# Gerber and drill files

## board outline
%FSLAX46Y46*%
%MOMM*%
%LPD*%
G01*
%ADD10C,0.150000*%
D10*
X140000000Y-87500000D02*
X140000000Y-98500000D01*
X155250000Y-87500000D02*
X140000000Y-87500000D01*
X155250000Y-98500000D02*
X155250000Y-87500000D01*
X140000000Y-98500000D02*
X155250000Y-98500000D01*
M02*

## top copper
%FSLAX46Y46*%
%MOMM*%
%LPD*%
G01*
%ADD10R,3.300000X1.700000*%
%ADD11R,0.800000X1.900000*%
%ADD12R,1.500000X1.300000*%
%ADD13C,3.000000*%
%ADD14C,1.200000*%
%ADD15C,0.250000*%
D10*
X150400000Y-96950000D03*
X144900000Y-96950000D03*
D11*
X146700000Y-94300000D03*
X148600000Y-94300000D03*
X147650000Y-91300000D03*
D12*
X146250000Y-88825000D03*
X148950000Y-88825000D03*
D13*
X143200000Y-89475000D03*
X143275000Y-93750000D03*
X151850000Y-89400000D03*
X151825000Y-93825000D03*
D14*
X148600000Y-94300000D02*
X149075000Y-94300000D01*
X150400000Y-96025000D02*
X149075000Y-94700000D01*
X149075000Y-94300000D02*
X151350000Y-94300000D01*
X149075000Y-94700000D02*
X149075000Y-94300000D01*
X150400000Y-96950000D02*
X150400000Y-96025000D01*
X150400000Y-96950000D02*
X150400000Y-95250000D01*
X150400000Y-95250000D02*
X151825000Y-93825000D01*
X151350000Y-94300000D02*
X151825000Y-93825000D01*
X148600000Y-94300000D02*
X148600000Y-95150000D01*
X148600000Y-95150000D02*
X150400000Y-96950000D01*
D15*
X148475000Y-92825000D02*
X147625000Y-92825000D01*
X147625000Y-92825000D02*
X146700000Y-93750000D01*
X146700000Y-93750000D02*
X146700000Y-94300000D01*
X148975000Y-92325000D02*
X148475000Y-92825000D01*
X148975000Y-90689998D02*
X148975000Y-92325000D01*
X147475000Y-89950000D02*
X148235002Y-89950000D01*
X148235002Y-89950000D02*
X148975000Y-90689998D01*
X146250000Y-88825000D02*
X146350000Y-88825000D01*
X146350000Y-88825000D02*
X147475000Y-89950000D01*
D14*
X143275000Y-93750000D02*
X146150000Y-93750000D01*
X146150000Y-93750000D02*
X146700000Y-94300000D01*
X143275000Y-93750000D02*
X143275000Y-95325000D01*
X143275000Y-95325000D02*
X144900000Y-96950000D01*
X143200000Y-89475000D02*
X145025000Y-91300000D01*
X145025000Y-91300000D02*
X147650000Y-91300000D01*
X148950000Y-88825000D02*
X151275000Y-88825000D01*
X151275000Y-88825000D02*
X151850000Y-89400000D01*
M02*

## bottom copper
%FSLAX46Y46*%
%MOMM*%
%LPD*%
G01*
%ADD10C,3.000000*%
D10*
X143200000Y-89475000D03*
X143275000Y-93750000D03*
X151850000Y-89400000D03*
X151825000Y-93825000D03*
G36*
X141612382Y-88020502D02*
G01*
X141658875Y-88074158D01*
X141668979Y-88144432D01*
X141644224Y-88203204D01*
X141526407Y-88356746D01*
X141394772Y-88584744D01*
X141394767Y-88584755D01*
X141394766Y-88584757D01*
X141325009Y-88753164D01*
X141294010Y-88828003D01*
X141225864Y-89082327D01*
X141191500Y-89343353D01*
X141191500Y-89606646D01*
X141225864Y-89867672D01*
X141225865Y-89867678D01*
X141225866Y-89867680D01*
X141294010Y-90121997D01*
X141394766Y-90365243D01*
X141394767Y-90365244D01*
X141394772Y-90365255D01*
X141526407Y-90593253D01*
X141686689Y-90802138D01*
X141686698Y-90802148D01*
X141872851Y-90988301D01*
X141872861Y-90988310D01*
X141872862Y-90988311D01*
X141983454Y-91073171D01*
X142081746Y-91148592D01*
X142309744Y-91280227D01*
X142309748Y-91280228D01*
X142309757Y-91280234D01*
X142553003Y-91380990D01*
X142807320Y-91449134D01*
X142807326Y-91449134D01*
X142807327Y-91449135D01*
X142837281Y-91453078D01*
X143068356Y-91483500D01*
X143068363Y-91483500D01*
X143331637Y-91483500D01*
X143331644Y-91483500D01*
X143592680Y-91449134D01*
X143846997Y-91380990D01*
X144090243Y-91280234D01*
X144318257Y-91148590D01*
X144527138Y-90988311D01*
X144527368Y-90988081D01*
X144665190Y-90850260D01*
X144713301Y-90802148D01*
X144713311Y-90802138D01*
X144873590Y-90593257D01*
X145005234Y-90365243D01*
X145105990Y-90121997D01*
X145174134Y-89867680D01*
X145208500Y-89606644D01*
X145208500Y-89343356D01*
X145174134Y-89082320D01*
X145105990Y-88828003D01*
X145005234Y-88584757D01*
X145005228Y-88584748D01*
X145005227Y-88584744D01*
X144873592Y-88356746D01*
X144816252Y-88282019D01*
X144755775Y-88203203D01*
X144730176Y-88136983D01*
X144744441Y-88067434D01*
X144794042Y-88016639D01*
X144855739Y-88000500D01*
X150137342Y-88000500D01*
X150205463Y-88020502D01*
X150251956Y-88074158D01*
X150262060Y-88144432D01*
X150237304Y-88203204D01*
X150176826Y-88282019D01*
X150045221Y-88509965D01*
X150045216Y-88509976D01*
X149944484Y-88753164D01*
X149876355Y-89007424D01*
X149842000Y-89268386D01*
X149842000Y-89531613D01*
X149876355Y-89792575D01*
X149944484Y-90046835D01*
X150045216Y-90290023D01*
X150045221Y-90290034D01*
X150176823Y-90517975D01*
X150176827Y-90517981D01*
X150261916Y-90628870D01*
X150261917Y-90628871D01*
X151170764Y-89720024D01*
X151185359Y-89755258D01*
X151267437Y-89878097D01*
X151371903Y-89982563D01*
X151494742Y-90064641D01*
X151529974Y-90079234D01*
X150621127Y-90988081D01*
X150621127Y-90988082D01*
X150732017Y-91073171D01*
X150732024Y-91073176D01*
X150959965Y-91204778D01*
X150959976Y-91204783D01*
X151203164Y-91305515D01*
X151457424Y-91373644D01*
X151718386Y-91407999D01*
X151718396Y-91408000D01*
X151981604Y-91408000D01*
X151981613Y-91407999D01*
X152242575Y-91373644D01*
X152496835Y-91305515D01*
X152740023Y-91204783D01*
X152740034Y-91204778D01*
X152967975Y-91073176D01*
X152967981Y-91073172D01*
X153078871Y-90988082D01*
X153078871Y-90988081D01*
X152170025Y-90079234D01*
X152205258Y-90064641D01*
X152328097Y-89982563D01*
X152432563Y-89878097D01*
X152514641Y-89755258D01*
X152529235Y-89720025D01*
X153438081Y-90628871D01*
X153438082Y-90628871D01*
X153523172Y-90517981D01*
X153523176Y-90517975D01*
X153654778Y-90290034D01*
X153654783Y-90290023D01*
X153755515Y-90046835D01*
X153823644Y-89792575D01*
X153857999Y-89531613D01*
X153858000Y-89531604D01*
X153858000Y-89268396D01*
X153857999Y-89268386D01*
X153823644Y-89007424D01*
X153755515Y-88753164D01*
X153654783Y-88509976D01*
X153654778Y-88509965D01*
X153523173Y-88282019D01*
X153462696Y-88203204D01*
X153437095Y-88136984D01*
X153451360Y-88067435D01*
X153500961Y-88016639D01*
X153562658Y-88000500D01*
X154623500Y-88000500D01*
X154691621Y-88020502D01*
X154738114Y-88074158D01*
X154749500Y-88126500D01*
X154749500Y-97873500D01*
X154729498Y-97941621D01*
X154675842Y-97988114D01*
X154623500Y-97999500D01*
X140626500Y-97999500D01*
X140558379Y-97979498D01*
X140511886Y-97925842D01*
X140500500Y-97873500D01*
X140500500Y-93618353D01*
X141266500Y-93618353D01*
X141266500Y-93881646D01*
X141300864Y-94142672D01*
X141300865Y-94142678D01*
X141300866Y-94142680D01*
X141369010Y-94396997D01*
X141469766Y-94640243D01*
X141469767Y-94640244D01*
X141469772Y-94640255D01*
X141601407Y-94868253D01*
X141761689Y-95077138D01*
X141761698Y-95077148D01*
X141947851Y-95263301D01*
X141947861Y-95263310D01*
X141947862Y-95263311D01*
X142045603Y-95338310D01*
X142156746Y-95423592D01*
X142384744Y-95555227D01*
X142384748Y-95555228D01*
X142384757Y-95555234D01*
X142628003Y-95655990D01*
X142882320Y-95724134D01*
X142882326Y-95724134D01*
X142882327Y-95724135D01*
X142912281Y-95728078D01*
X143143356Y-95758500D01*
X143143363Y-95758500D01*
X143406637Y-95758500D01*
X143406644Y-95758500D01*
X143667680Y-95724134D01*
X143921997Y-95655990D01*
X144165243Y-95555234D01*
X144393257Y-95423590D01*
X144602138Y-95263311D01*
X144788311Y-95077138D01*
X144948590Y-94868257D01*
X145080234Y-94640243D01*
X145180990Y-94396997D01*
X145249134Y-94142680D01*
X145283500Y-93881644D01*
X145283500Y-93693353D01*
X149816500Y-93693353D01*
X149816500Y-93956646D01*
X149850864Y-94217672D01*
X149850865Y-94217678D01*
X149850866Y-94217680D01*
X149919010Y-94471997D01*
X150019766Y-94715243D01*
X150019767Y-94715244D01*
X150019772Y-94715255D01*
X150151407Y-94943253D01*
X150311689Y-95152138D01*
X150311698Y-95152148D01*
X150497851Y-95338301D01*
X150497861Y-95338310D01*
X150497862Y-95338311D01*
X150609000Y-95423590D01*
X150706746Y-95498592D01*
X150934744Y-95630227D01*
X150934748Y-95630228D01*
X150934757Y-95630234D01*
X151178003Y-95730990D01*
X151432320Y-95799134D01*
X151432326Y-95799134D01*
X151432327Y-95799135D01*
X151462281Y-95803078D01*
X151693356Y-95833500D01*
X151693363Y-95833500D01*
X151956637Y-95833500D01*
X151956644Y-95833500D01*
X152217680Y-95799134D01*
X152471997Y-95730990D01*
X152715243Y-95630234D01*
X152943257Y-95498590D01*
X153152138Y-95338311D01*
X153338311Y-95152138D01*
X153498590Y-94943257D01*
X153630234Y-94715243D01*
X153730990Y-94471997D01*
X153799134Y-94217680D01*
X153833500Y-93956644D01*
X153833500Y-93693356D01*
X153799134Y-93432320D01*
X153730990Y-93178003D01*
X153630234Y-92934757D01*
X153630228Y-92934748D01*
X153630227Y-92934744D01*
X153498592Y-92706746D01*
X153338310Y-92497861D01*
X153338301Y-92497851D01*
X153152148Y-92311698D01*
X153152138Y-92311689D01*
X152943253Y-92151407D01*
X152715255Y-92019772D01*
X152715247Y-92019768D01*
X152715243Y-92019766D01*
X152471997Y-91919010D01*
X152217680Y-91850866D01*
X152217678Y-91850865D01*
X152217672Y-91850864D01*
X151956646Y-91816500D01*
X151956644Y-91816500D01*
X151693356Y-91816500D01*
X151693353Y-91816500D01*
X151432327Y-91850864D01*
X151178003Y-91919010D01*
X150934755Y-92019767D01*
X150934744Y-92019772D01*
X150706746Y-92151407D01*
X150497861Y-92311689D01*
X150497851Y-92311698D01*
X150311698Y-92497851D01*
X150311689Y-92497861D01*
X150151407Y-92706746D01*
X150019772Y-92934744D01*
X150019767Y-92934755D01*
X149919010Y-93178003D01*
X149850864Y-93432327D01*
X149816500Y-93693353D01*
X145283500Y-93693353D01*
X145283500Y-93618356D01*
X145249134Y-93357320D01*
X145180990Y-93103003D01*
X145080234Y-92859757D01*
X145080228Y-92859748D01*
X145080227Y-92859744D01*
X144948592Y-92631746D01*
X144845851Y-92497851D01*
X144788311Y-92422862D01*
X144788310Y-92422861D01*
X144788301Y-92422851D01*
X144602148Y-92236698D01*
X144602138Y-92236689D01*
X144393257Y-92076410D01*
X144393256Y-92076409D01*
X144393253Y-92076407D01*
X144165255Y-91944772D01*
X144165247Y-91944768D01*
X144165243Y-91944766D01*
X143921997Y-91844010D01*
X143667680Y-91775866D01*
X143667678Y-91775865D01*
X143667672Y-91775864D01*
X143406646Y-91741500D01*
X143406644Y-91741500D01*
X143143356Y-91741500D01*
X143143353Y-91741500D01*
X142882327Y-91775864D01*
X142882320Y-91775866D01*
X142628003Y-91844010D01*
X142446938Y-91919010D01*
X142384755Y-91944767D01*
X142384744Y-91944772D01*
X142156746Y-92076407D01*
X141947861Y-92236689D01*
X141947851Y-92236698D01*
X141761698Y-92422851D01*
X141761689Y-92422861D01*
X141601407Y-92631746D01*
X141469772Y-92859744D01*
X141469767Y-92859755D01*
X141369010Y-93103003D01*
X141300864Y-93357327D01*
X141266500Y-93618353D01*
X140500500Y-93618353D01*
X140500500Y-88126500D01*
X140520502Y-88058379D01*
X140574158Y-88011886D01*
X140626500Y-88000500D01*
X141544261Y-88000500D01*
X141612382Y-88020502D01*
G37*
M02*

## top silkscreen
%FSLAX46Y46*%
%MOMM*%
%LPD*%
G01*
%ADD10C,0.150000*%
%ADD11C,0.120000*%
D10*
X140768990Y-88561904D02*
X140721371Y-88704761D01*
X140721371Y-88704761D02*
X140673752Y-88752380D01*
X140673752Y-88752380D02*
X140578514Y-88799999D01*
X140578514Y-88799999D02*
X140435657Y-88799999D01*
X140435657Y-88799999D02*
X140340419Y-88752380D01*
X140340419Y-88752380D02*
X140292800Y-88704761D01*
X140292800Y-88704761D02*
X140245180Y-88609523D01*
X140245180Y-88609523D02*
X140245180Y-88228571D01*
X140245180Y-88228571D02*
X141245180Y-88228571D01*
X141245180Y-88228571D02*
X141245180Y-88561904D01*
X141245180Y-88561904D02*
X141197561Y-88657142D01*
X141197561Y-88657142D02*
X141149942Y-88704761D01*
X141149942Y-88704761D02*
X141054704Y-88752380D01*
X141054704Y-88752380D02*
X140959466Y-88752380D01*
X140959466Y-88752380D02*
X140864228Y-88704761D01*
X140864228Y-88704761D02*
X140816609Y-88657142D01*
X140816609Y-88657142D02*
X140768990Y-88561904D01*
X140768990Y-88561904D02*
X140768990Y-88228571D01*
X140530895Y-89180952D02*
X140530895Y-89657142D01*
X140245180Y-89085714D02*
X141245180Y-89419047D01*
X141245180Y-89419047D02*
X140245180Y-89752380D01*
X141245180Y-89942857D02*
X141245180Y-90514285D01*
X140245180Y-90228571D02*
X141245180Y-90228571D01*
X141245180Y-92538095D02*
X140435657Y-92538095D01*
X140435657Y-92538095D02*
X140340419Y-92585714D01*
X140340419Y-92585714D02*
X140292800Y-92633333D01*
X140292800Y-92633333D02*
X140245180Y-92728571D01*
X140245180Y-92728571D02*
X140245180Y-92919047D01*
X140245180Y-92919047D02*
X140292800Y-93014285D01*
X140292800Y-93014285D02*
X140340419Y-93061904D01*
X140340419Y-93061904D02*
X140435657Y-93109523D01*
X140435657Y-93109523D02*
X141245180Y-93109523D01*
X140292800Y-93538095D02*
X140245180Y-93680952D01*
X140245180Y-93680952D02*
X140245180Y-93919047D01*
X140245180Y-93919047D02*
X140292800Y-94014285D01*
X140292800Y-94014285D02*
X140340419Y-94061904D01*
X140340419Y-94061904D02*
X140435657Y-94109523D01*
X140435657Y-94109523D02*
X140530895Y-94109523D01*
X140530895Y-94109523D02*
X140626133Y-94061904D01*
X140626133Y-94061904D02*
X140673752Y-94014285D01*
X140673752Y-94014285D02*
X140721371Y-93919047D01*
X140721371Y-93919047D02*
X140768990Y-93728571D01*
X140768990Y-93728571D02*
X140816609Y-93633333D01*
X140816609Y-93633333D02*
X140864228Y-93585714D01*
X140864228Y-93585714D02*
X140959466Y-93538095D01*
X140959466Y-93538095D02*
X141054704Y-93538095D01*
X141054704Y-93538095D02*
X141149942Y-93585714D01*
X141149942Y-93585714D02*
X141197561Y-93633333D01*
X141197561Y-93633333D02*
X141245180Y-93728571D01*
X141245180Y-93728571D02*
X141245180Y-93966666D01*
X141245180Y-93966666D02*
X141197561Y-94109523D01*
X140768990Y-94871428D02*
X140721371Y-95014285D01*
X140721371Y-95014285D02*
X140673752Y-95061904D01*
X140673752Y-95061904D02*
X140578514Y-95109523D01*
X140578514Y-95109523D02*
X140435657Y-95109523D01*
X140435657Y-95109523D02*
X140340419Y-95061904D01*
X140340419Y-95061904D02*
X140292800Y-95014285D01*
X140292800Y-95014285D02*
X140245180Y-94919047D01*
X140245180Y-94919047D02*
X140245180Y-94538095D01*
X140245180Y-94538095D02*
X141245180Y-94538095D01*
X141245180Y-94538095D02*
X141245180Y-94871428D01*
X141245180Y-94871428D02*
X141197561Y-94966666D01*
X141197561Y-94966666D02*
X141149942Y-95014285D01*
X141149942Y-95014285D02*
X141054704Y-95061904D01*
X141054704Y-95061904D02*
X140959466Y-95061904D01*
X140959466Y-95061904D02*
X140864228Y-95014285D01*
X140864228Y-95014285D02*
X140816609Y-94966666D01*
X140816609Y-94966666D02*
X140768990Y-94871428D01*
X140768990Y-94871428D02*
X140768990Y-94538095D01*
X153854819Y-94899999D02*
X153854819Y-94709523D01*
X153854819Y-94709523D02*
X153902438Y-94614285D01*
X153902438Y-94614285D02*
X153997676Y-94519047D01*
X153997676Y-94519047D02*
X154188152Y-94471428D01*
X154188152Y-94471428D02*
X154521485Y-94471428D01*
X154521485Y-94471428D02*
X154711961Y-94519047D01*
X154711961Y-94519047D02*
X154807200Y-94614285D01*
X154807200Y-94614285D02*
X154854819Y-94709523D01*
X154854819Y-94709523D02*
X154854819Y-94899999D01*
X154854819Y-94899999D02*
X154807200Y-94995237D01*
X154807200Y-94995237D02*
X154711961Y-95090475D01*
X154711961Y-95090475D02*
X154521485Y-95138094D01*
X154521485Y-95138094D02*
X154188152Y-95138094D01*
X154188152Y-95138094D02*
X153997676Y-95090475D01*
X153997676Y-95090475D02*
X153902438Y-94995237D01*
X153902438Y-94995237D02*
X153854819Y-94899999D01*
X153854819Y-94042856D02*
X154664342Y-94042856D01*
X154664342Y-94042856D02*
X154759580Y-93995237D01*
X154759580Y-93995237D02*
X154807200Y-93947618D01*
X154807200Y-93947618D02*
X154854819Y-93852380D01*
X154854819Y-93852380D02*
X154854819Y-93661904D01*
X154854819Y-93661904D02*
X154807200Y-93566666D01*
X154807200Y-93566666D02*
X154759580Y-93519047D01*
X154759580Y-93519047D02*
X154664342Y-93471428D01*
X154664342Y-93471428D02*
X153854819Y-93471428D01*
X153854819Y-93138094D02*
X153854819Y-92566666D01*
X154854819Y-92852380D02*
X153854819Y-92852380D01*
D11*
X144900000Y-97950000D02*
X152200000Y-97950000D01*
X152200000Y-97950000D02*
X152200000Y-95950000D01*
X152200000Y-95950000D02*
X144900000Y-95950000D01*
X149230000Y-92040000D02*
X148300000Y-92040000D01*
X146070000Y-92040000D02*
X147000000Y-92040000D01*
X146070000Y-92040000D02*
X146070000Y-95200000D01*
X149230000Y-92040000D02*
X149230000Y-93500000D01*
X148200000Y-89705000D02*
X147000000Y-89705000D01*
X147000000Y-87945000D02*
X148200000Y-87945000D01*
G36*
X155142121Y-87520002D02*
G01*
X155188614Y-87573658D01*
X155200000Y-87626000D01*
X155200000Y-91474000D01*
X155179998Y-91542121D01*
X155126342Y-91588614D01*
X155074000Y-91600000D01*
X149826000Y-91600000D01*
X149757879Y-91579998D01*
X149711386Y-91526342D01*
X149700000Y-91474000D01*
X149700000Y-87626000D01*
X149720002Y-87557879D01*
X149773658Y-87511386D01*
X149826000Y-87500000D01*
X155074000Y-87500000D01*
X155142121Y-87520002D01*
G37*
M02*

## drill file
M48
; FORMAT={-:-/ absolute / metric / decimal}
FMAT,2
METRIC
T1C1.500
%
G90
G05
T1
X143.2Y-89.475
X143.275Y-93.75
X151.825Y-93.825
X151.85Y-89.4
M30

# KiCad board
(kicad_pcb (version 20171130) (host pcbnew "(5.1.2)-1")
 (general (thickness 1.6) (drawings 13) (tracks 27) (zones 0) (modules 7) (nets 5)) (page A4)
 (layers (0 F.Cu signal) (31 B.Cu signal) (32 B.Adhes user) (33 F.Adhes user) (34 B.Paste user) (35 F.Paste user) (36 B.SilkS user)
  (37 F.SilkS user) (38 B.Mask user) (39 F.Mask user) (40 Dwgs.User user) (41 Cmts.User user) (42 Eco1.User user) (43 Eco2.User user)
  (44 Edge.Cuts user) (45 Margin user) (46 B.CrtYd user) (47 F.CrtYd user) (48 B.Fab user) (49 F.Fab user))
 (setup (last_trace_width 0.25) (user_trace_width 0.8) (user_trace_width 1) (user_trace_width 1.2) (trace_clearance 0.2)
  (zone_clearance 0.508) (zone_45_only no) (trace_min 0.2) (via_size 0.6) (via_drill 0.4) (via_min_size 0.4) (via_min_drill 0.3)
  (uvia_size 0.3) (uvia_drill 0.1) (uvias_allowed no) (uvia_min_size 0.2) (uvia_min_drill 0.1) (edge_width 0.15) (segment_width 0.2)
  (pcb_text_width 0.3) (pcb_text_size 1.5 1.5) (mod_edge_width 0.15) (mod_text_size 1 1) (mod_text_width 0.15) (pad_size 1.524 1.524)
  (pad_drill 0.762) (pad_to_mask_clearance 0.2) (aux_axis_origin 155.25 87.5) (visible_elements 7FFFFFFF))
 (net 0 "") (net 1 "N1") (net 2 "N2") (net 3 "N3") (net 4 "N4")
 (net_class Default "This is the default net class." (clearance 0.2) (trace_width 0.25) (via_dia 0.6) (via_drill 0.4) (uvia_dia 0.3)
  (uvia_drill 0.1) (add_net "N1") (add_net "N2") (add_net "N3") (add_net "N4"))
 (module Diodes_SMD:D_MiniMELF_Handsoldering (layer F.Cu) (at 147.65 96.95 180)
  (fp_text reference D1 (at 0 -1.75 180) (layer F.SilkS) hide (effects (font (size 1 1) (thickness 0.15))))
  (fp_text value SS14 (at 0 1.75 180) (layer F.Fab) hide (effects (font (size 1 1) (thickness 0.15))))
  (fp_line (start 2.75 -1) (end -4.55 -1) (layer F.SilkS) (width 0.12))
  (fp_line (start -4.55 -1) (end -4.55 1) (layer F.SilkS) (width 0.12))
  (fp_line (start -4.55 1) (end 2.75 1) (layer F.SilkS) (width 0.12))
  (pad 1 smd rect (at -2.75 0 180) (size 3.3 1.7) (layers F.Cu F.Paste F.Mask) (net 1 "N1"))
  (pad 2 smd rect (at 2.75 0 180) (size 3.3 1.7) (layers F.Cu F.Paste F.Mask) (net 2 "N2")))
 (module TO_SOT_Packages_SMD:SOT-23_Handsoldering (layer F.Cu) (at 147.65 92.8 90)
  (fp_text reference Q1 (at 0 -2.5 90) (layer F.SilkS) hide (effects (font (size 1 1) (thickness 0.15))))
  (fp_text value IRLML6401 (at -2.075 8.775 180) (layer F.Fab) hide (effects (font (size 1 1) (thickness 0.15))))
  (fp_line (start 0.76 1.58) (end 0.76 0.65) (layer F.SilkS) (width 0.12))
  (fp_line (start 0.76 -1.58) (end 0.76 -0.65) (layer F.SilkS) (width 0.12))
  (fp_line (start 0.76 -1.58) (end -2.4 -1.58) (layer F.SilkS) (width 0.12))
  (fp_line (start 0.76 1.58) (end -0.7 1.58) (layer F.SilkS) (width 0.12))
  (pad 1 smd rect (at -1.5 -0.95 90) (size 1.9 0.8) (layers F.Cu F.Paste F.Mask) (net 2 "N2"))
  (pad 2 smd rect (at -1.5 0.95 90) (size 1.9 0.8) (layers F.Cu F.Paste F.Mask) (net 1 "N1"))
  (pad 3 smd rect (at 1.5 0 90) (size 1.9 0.8) (layers F.Cu F.Paste F.Mask) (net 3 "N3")))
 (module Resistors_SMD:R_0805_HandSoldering (layer F.Cu) (at 147.6 88.825)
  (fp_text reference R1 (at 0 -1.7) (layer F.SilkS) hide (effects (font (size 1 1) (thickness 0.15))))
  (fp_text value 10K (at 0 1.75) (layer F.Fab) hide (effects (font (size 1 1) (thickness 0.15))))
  (fp_line (start 0.6 0.88) (end -0.6 0.88) (layer F.SilkS) (width 0.12))
  (fp_line (start -0.6 -0.88) (end 0.6 -0.88) (layer F.SilkS) (width 0.12))
  (pad 1 smd rect (at -1.35 0) (size 1.5 1.3) (layers F.Cu F.Paste F.Mask) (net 2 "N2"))
  (pad 2 smd rect (at 1.35 0) (size 1.5 1.3) (layers F.Cu F.Paste F.Mask) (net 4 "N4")))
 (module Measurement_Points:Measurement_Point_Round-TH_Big (layer F.Cu) (at 143.2 89.475)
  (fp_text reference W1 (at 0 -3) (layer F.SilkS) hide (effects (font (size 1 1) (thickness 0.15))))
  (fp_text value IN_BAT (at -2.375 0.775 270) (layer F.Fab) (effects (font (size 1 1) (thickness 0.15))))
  (pad 1 thru_hole circle (at 0 0) (size 3 3) (drill 1.5) (layers *.Cu *.Mask) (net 3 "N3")))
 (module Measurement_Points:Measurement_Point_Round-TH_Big (layer F.Cu) (at 143.275 93.75)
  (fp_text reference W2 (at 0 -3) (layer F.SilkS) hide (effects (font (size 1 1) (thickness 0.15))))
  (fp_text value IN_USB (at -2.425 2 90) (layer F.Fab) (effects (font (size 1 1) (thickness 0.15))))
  (pad 1 thru_hole circle (at 0 0) (size 3 3) (drill 1.5) (layers *.Cu *.Mask) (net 2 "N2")))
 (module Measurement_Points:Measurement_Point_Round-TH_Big (layer F.Cu) (at 151.85 89.4)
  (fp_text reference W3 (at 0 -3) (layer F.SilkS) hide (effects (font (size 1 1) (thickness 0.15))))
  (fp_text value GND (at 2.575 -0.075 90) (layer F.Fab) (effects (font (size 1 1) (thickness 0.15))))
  (pad 1 thru_hole circle (at 0 0) (size 3 3) (drill 1.5) (layers *.Cu *.Mask) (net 4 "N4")))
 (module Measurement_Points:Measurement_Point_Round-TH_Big (layer F.Cu) (at 151.825 93.825)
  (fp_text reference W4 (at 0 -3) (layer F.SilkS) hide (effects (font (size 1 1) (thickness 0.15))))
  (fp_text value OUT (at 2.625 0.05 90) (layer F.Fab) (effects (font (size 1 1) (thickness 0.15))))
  (pad 1 thru_hole circle (at 0 0) (size 3 3) (drill 1.5) (layers *.Cu *.Mask) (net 1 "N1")))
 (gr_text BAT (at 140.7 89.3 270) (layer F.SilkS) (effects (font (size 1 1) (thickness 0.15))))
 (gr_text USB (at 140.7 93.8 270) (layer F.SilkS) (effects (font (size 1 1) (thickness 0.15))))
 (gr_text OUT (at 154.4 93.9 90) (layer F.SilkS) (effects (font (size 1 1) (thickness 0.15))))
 (gr_line (start 140 87.5) (end 140 98.5) (layer Edge.Cuts) (width 0.15))
 (gr_line (start 155.25 87.5) (end 140 87.5) (layer Edge.Cuts) (width 0.15))
 (gr_line (start 155.25 98.5) (end 155.25 87.5) (layer Edge.Cuts) (width 0.15))
 (gr_line (start 140 98.5) (end 155.25 98.5) (layer Edge.Cuts) (width 0.15))
 (segment (start 148.6 94.3) (end 149.075 94.3) (width 1.2) (layer F.Cu) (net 1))
 (segment (start 150.4 96.025) (end 149.075 94.7) (width 1.2) (layer F.Cu) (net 1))
 (segment (start 149.075 94.3) (end 151.35 94.3) (width 1.2) (layer F.Cu) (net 1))
 (segment (start 149.075 94.7) (end 149.075 94.3) (width 1.2) (layer F.Cu) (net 1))
 (segment (start 150.4 96.95) (end 150.4 96.025) (width 1.2) (layer F.Cu) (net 1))
 (segment (start 150.4 96.95) (end 150.4 95.25) (width 1.2) (layer F.Cu) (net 1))
 (segment (start 150.4 95.25) (end 151.825 93.825) (width 1.2) (layer F.Cu) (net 1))
 (segment (start 151.35 94.3) (end 151.825 93.825) (width 1.2) (layer F.Cu) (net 1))
 (segment (start 148.6 94.3) (end 148.6 95.15) (width 1.2) (layer F.Cu) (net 1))
 (segment (start 148.6 95.15) (end 150.4 96.95) (width 1.2) (layer F.Cu) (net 1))
 (segment (start 148.475 92.825) (end 147.625 92.825) (width 0.25) (layer F.Cu) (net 2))
 (segment (start 147.625 92.825) (end 146.7 93.75) (width 0.25) (layer F.Cu) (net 2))
 (segment (start 146.7 93.75) (end 146.7 94.3) (width 0.25) (layer F.Cu) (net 2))
 (segment (start 148.975 92.325) (end 148.475 92.825) (width 0.25) (layer F.Cu) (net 2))
 (segment (start 148.975 90.689998) (end 148.975 92.325) (width 0.25) (layer F.Cu) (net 2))
 (segment (start 147.475 89.95) (end 148.235002 89.95) (width 0.25) (layer F.Cu) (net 2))
 (segment (start 148.235002 89.95) (end 148.975 90.689998) (width 0.25) (layer F.Cu) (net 2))
 (segment (start 146.25 88.825) (end 146.35 88.825) (width 0.25) (layer F.Cu) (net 2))
 (segment (start 146.35 88.825) (end 147.475 89.95) (width 0.25) (layer F.Cu) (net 2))
 (segment (start 143.275 93.75) (end 146.15 93.75) (width 1.2) (layer F.Cu) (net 2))
 (segment (start 146.15 93.75) (end 146.7 94.3) (width 1.2) (layer F.Cu) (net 2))
 (segment (start 143.275 93.75) (end 143.275 95.325) (width 1.2) (layer F.Cu) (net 2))
 (segment (start 143.275 95.325) (end 144.9 96.95) (width 1.2) (layer F.Cu) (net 2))
 (segment (start 143.2 89.475) (end 145.025 91.3) (width 1.2) (layer F.Cu) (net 3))
 (segment (start 145.025 91.3) (end 147.65 91.3) (width 1.2) (layer F.Cu) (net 3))
 (segment (start 148.95 88.825) (end 151.275 88.825) (width 1.2) (layer F.Cu) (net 4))
 (segment (start 151.275 88.825) (end 151.85 89.4) (width 1.2) (layer F.Cu) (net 4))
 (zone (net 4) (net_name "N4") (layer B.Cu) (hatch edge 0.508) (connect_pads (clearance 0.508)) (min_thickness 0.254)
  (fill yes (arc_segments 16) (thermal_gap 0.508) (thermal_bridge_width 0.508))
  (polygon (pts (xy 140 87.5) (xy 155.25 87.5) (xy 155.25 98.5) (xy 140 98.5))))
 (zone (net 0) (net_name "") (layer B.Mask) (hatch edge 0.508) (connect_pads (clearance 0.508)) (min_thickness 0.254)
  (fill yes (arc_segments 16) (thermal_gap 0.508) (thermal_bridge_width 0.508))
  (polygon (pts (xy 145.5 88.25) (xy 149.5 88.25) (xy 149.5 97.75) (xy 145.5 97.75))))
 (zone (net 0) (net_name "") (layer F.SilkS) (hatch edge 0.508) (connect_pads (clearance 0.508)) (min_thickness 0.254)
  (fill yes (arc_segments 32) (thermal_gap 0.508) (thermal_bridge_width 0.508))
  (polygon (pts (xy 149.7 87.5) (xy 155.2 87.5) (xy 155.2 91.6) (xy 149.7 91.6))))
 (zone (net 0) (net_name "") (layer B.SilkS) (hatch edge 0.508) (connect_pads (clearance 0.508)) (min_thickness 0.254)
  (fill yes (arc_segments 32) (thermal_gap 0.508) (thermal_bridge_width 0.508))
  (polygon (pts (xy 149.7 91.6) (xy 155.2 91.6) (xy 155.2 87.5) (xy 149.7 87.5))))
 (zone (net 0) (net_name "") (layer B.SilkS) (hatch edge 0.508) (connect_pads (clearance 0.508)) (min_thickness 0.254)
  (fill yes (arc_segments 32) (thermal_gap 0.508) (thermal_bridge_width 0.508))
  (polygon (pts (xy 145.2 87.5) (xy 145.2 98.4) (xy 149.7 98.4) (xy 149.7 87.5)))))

